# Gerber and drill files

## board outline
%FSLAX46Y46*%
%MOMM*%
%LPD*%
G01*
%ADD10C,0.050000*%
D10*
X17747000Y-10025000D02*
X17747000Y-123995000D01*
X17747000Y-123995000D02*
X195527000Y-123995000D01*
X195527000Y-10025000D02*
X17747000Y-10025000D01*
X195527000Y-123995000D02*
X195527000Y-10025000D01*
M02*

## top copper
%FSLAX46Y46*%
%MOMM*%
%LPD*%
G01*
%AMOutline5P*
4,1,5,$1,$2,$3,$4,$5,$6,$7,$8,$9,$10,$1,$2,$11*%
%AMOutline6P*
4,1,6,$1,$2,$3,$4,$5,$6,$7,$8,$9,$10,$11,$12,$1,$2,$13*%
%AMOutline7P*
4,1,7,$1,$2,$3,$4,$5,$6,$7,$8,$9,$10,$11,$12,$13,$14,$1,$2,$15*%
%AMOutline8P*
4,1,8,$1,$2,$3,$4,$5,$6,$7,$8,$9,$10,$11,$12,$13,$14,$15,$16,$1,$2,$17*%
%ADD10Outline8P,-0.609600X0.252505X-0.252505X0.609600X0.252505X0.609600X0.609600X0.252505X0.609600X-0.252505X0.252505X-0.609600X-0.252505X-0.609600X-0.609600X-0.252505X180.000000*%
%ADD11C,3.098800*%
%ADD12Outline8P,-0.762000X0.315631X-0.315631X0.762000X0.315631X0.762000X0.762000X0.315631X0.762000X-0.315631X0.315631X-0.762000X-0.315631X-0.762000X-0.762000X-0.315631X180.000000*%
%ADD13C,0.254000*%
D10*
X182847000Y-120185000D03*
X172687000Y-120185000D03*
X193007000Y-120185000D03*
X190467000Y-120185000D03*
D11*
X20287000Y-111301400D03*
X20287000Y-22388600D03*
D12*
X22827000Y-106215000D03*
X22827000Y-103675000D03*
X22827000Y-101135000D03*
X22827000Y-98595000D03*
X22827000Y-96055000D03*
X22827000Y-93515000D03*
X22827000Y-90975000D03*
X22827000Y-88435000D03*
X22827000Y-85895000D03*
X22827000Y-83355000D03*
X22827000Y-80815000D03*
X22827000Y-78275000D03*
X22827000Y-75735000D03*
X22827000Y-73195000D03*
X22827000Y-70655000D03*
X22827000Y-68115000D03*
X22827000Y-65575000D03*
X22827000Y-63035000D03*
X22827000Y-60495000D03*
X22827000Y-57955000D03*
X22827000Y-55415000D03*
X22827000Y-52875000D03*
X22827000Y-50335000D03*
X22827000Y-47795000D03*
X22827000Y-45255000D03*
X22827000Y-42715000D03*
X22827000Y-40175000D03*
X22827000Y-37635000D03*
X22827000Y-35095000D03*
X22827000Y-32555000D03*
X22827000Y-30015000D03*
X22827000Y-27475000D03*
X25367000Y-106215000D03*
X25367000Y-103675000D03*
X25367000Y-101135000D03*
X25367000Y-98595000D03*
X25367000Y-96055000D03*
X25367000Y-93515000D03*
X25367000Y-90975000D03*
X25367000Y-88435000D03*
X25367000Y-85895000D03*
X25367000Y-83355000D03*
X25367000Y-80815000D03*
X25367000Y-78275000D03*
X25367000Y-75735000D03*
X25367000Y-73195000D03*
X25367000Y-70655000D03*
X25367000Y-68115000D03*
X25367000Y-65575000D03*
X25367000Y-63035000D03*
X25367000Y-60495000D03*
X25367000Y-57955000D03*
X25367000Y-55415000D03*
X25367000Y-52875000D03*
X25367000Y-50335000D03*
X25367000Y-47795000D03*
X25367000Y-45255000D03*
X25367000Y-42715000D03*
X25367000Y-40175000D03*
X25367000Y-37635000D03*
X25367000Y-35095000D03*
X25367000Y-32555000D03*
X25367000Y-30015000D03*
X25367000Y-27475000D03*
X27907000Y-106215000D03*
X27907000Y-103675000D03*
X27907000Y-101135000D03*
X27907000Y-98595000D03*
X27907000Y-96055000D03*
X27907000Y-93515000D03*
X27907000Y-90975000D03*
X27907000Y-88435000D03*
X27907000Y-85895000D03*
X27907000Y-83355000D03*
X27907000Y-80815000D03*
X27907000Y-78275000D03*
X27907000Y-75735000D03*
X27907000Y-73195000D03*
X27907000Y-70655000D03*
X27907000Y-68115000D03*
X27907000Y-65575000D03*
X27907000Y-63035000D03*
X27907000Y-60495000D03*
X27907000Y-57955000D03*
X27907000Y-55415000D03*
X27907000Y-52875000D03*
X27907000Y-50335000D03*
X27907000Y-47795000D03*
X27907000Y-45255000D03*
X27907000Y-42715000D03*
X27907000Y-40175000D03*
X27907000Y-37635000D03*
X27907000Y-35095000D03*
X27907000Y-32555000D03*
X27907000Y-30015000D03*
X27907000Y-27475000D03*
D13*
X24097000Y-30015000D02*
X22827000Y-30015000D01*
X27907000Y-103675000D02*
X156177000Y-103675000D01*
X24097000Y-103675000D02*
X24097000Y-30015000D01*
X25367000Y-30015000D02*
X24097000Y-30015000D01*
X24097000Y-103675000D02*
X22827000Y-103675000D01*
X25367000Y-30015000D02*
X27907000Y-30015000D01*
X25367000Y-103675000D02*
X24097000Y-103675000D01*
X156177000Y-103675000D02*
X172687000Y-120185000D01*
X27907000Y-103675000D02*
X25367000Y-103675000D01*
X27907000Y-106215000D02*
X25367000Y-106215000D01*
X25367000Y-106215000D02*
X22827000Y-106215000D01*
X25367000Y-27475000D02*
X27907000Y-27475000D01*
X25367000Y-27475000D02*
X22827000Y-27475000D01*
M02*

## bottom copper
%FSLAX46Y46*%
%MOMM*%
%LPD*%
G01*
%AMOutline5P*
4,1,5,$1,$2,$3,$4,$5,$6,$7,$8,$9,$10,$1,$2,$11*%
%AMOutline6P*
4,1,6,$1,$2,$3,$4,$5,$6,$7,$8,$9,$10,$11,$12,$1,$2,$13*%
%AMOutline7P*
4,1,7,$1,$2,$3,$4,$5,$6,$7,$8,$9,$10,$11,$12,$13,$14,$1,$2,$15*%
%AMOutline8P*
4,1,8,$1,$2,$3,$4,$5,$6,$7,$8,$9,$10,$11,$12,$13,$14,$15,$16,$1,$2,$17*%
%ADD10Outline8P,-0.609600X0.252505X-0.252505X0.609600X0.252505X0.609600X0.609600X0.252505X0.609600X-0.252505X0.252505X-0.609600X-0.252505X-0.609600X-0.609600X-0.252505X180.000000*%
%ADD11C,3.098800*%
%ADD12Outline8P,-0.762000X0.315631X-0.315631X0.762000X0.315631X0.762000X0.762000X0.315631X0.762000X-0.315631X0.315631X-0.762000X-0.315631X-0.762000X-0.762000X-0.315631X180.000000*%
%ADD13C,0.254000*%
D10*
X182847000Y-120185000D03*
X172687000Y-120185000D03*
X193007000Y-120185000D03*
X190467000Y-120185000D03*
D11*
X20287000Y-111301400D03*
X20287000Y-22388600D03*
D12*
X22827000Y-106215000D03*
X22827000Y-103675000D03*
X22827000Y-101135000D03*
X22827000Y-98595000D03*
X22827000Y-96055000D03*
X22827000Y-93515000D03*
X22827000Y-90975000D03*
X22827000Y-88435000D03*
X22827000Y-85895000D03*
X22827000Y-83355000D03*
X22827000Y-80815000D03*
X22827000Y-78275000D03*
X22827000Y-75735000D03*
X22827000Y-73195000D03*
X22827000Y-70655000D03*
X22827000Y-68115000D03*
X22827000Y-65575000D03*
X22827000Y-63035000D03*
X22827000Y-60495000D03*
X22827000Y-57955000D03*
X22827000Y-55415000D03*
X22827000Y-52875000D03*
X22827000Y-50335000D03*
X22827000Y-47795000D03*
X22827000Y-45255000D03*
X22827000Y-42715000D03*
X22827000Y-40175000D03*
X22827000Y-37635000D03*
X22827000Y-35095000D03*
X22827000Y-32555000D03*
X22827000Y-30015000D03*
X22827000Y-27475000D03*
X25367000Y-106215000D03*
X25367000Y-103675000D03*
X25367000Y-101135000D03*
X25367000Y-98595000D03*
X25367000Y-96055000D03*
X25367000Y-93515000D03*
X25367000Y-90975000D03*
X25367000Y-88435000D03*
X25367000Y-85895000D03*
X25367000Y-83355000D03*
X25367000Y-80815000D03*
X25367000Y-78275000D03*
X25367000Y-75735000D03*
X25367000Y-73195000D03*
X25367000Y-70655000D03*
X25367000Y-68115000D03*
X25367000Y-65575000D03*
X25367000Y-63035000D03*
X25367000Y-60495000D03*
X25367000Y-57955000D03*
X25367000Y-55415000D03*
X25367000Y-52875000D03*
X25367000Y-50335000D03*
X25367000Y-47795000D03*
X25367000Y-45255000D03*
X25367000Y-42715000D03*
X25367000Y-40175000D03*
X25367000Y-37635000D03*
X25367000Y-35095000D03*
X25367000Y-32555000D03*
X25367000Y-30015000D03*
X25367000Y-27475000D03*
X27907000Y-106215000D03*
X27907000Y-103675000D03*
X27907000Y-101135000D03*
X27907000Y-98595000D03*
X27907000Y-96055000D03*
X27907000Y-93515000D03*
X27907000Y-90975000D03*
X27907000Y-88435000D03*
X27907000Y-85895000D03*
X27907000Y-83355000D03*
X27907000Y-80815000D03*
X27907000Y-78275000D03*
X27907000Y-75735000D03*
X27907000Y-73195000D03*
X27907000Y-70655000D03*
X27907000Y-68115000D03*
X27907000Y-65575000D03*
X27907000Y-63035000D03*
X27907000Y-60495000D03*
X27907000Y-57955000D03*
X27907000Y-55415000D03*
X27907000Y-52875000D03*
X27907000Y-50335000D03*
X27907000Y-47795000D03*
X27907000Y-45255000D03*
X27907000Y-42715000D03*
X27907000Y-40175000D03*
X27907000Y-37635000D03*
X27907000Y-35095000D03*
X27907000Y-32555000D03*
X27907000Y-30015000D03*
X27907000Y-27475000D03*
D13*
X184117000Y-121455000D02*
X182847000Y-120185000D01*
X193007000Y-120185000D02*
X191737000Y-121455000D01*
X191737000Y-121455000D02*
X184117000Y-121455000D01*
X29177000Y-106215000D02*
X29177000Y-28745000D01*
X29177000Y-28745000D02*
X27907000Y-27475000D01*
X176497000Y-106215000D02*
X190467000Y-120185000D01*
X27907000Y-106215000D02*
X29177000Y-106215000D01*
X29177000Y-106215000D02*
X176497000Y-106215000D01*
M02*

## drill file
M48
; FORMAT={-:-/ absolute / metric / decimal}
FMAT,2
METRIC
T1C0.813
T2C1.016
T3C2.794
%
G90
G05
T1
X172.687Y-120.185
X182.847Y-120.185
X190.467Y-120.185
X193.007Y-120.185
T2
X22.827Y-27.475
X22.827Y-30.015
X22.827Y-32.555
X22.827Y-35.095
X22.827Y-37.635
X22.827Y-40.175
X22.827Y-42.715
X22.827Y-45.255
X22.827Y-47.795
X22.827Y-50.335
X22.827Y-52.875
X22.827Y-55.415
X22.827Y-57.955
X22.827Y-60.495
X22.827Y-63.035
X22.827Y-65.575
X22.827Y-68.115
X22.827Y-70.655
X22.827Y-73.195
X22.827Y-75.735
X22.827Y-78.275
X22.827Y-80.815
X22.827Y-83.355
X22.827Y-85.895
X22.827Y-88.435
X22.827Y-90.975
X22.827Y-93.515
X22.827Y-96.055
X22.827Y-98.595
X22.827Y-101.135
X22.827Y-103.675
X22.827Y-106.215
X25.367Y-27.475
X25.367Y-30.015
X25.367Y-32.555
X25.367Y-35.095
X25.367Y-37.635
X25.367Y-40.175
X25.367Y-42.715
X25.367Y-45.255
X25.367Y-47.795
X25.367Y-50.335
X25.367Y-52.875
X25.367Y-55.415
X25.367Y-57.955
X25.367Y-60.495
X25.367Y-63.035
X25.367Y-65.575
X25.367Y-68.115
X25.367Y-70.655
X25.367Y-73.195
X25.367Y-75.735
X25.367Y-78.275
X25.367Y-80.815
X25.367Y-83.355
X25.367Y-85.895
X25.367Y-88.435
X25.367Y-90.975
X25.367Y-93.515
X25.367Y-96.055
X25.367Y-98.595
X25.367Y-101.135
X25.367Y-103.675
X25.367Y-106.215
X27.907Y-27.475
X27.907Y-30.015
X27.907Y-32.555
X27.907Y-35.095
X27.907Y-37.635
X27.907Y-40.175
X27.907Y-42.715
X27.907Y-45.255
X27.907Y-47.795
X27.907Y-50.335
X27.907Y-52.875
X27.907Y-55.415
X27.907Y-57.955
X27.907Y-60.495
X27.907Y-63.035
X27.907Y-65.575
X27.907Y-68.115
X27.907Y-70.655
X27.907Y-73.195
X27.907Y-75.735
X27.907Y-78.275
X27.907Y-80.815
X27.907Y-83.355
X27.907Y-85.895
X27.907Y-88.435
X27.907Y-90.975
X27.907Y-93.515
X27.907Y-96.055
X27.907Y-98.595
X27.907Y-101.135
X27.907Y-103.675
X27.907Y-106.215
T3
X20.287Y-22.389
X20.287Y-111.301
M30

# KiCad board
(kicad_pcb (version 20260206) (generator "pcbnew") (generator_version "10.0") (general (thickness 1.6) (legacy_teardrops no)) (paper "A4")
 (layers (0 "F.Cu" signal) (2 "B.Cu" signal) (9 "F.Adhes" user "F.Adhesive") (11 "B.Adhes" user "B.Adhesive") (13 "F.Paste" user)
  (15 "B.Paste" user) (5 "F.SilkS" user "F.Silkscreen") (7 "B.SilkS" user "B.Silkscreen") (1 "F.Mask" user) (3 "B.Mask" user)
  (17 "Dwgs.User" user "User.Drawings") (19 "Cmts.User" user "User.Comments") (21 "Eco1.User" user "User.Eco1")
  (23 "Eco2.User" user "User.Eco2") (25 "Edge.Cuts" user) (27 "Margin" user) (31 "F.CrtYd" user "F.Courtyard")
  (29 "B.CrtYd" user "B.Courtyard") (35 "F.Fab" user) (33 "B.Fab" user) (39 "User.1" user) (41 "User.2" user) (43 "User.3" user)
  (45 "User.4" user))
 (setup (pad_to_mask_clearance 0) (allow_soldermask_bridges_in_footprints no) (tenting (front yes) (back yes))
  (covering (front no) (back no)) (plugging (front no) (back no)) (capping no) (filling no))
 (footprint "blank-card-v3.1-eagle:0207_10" (layer "F.Cu") (at 177.767 120.185 180)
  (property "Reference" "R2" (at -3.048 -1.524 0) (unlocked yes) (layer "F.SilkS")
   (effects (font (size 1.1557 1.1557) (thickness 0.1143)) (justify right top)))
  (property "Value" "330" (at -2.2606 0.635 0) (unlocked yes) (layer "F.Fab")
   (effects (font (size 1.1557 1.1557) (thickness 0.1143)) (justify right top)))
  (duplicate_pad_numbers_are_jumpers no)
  (pad "1" thru_hole roundrect (at -5.08 0 180) (size 1.2192 1.2192) (drill 0.8128) (layers "*.Cu" "*.Mask") (remove_unused_layers no)
   (roundrect_rratio 0.25) (chamfer_ratio 0.2928932188) (chamfer top_left top_right bottom_left bottom_right) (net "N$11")
   (solder_mask_margin 0.0635) (thermal_bridge_angle 0))
  (pad "2" thru_hole roundrect (at 5.08 0 180) (size 1.2192 1.2192) (drill 0.8128) (layers "*.Cu" "*.Mask") (remove_unused_layers no)
   (roundrect_rratio 0.25) (chamfer_ratio 0.2928932188) (chamfer top_left top_right bottom_left bottom_right) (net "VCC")
   (solder_mask_margin 0.0635) (thermal_bridge_angle 0)))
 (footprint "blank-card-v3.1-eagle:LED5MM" (layer "F.Cu") (at 191.737 120.185 180)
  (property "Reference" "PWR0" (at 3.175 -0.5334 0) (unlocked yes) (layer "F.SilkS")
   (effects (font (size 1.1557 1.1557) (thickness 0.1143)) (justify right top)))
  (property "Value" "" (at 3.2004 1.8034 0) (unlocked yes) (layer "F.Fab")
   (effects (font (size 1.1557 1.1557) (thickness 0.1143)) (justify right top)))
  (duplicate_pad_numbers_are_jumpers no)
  (pad "A" thru_hole roundrect (at -1.27 0 180) (size 1.2192 1.2192) (drill 0.8128) (layers "*.Cu" "*.Mask") (remove_unused_layers no)
   (roundrect_rratio 0.25) (chamfer_ratio 0.2928932188) (chamfer top_left top_right bottom_left bottom_right) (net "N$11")
   (solder_mask_margin 0.0635) (thermal_bridge_angle 0))
  (pad "K" thru_hole roundrect (at 1.27 0 180) (size 1.2192 1.2192) (drill 0.8128) (layers "*.Cu" "*.Mask") (remove_unused_layers no)
   (roundrect_rratio 0.25) (chamfer_ratio 0.2928932188) (chamfer top_left top_right bottom_left bottom_right) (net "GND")
   (solder_mask_margin 0.0635) (thermal_bridge_angle 0)))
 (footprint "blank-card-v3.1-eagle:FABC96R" (layer "F.Cu") (at 20.287 66.845 180)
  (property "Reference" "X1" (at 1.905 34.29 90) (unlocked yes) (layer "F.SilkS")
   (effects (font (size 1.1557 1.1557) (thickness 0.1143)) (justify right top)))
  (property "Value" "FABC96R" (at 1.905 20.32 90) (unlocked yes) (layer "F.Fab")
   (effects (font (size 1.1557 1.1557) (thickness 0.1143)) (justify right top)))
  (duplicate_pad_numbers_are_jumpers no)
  (pad "" np_thru_hole circle (at 0 -44.4564 180) (size 3.0988 3.0988) (drill 2.794) (layers "*.Cu" "*.Mask"))
  (pad "" np_thru_hole circle (at 0 44.4564 180) (size 3.0988 3.0988) (drill 2.794) (layers "*.Cu" "*.Mask"))
  (pad "A1" thru_hole roundrect (at -2.54 -39.37 180) (size 1.524 1.524) (drill 1.016) (layers "*.Cu" "*.Mask") (remove_unused_layers no)
   (roundrect_rratio 0.25) (chamfer_ratio 0.2928932188) (chamfer top_left top_right bottom_left bottom_right) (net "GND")
   (solder_mask_margin 0.0635) (thermal_bridge_angle 0))
  (pad "A2" thru_hole roundrect (at -2.54 -36.83 180) (size 1.524 1.524) (drill 1.016) (layers "*.Cu" "*.Mask") (remove_unused_layers no)
   (roundrect_rratio 0.25) (chamfer_ratio 0.2928932188) (chamfer top_left top_right bottom_left bottom_right) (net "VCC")
   (solder_mask_margin 0.0635) (thermal_bridge_angle 0))
  (pad "A3" thru_hole roundrect (at -2.54 -34.29 180) (size 1.524 1.524) (drill 1.016) (layers "*.Cu" "*.Mask") (remove_unused_layers no)
   (roundrect_rratio 0.25) (chamfer_ratio 0.2928932188) (chamfer top_left top_right bottom_left bottom_right) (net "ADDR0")
   (solder_mask_margin 0.0635) (thermal_bridge_angle 0))
  (pad "A4" thru_hole roundrect (at -2.54 -31.75 180) (size 1.524 1.524) (drill 1.016) (layers "*.Cu" "*.Mask") (remove_unused_layers no)
   (roundrect_rratio 0.25) (chamfer_ratio 0.2928932188) (chamfer top_left top_right bottom_left bottom_right) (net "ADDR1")
   (solder_mask_margin 0.0635) (thermal_bridge_angle 0))
  (pad "A5" thru_hole roundrect (at -2.54 -29.21 180) (size 1.524 1.524) (drill 1.016) (layers "*.Cu" "*.Mask") (remove_unused_layers no)
   (roundrect_rratio 0.25) (chamfer_ratio 0.2928932188) (chamfer top_left top_right bottom_left bottom_right) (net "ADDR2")
   (solder_mask_margin 0.0635) (thermal_bridge_angle 0))
  (pad "A6" thru_hole roundrect (at -2.54 -26.67 180) (size 1.524 1.524) (drill 1.016) (layers "*.Cu" "*.Mask") (remove_unused_layers no)
   (roundrect_rratio 0.25) (chamfer_ratio 0.2928932188) (chamfer top_left top_right bottom_left bottom_right) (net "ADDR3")
   (solder_mask_margin 0.0635) (thermal_bridge_angle 0))
  (pad "A7" thru_hole roundrect (at -2.54 -24.13 180) (size 1.524 1.524) (drill 1.016) (layers "*.Cu" "*.Mask") (remove_unused_layers no)
   (roundrect_rratio 0.25) (chamfer_ratio 0.2928932188) (chamfer top_left top_right bottom_left bottom_right) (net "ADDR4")
   (solder_mask_margin 0.0635) (thermal_bridge_angle 0))
  (pad "A8" thru_hole roundrect (at -2.54 -21.59 180) (size 1.524 1.524) (drill 1.016) (layers "*.Cu" "*.Mask") (remove_unused_layers no)
   (roundrect_rratio 0.25) (chamfer_ratio 0.2928932188) (chamfer top_left top_right bottom_left bottom_right) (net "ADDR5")
   (solder_mask_margin 0.0635) (thermal_bridge_angle 0))
  (pad "A9" thru_hole roundrect (at -2.54 -19.05 180) (size 1.524 1.524) (drill 1.016) (layers "*.Cu" "*.Mask") (remove_unused_layers no)
   (roundrect_rratio 0.25) (chamfer_ratio 0.2928932188) (chamfer top_left top_right bottom_left bottom_right) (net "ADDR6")
   (solder_mask_margin 0.0635) (thermal_bridge_angle 0))
  (pad "A10" thru_hole roundrect (at -2.54 -16.51 180) (size 1.524 1.524) (drill 1.016) (layers "*.Cu" "*.Mask") (remove_unused_layers no)
   (roundrect_rratio 0.25) (chamfer_ratio 0.2928932188) (chamfer top_left top_right bottom_left bottom_right) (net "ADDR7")
   (solder_mask_margin 0.0635) (thermal_bridge_angle 0))
  (pad "A11" thru_hole roundrect (at -2.54 -13.97 180) (size 1.524 1.524) (drill 1.016) (layers "*.Cu" "*.Mask") (remove_unused_layers no)
   (roundrect_rratio 0.25) (chamfer_ratio 0.2928932188) (chamfer top_left top_right bottom_left bottom_right) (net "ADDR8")
   (solder_mask_margin 0.0635) (thermal_bridge_angle 0))
  (pad "A12" thru_hole roundrect (at -2.54 -11.43 180) (size 1.524 1.524) (drill 1.016) (layers "*.Cu" "*.Mask") (remove_unused_layers no)
   (roundrect_rratio 0.25) (chamfer_ratio 0.2928932188) (chamfer top_left top_right bottom_left bottom_right) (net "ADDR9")
   (solder_mask_margin 0.0635) (thermal_bridge_angle 0))
  (pad "A13" thru_hole roundrect (at -2.54 -8.89 180) (size 1.524 1.524) (drill 1.016) (layers "*.Cu" "*.Mask") (remove_unused_layers no)
   (roundrect_rratio 0.25) (chamfer_ratio 0.2928932188) (chamfer top_left top_right bottom_left bottom_right) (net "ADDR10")
   (solder_mask_margin 0.0635) (thermal_bridge_angle 0))
  (pad "A14" thru_hole roundrect (at -2.54 -6.35 180) (size 1.524 1.524) (drill 1.016) (layers "*.Cu" "*.Mask") (remove_unused_layers no)
   (roundrect_rratio 0.25) (chamfer_ratio 0.2928932188) (chamfer top_left top_right bottom_left bottom_right) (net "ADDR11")
   (solder_mask_margin 0.0635) (thermal_bridge_angle 0))
  (pad "A15" thru_hole roundrect (at -2.54 -3.81 180) (size 1.524 1.524) (drill 1.016) (layers "*.Cu" "*.Mask") (remove_unused_layers no)
   (roundrect_rratio 0.25) (chamfer_ratio 0.2928932188) (chamfer top_left top_right bottom_left bottom_right) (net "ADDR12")
   (solder_mask_margin 0.0635) (thermal_bridge_angle 0))
  (pad "A16" thru_hole roundrect (at -2.54 -1.27 180) (size 1.524 1.524) (drill 1.016) (layers "*.Cu" "*.Mask") (remove_unused_layers no)
   (roundrect_rratio 0.25) (chamfer_ratio 0.2928932188) (chamfer top_left top_right bottom_left bottom_right) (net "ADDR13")
   (solder_mask_margin 0.0635) (thermal_bridge_angle 0))
  (pad "A17" thru_hole roundrect (at -2.54 1.27 180) (size 1.524 1.524) (drill 1.016) (layers "*.Cu" "*.Mask") (remove_unused_layers no)
   (roundrect_rratio 0.25) (chamfer_ratio 0.2928932188) (chamfer top_left top_right bottom_left bottom_right) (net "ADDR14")
   (solder_mask_margin 0.0635) (thermal_bridge_angle 0))
  (pad "A18" thru_hole roundrect (at -2.54 3.81 180) (size 1.524 1.524) (drill 1.016) (layers "*.Cu" "*.Mask") (remove_unused_layers no)
   (roundrect_rratio 0.25) (chamfer_ratio 0.2928932188) (chamfer top_left top_right bottom_left bottom_right) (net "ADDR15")
   (solder_mask_margin 0.0635) (thermal_bridge_angle 0))
  (pad "A19" thru_hole roundrect (at -2.54 6.35 180) (size 1.524 1.524) (drill 1.016) (layers "*.Cu" "*.Mask") (remove_unused_layers no)
   (roundrect_rratio 0.25) (chamfer_ratio 0.2928932188) (chamfer top_left top_right bottom_left bottom_right) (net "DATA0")
   (solder_mask_margin 0.0635) (thermal_bridge_angle 0))
  (pad "A20" thru_hole roundrect (at -2.54 8.89 180) (size 1.524 1.524) (drill 1.016) (layers "*.Cu" "*.Mask") (remove_unused_layers no)
   (roundrect_rratio 0.25) (chamfer_ratio 0.2928932188) (chamfer top_left top_right bottom_left bottom_right) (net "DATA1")
   (solder_mask_margin 0.0635) (thermal_bridge_angle 0))
  (pad "A21" thru_hole roundrect (at -2.54 11.43 180) (size 1.524 1.524) (drill 1.016) (layers "*.Cu" "*.Mask") (remove_unused_layers no)
   (roundrect_rratio 0.25) (chamfer_ratio 0.2928932188) (chamfer top_left top_right bottom_left bottom_right) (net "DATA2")
   (solder_mask_margin 0.0635) (thermal_bridge_angle 0))
  (pad "A22" thru_hole roundrect (at -2.54 13.97 180) (size 1.524 1.524) (drill 1.016) (layers "*.Cu" "*.Mask") (remove_unused_layers no)
   (roundrect_rratio 0.25) (chamfer_ratio 0.2928932188) (chamfer top_left top_right bottom_left bottom_right) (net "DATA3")
   (solder_mask_margin 0.0635) (thermal_bridge_angle 0))
  (pad "A23" thru_hole roundrect (at -2.54 16.51 180) (size 1.524 1.524) (drill 1.016) (layers "*.Cu" "*.Mask") (remove_unused_layers no)
   (roundrect_rratio 0.25) (chamfer_ratio 0.2928932188) (chamfer top_left top_right bottom_left bottom_right) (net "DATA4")
   (solder_mask_margin 0.0635) (thermal_bridge_angle 0))
  (pad "A24" thru_hole roundrect (at -2.54 19.05 180) (size 1.524 1.524) (drill 1.016) (layers "*.Cu" "*.Mask") (remove_unused_layers no)
   (roundrect_rratio 0.25) (chamfer_ratio 0.2928932188) (chamfer top_left top_right bottom_left bottom_right) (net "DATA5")
   (solder_mask_margin 0.0635) (thermal_bridge_angle 0))
  (pad "A25" thru_hole roundrect (at -2.54 21.59 180) (size 1.524 1.524) (drill 1.016) (layers "*.Cu" "*.Mask") (remove_unused_layers no)
   (roundrect_rratio 0.25) (chamfer_ratio 0.2928932188) (chamfer top_left top_right bottom_left bottom_right) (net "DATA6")
   (solder_mask_margin 0.0635) (thermal_bridge_angle 0))
  (pad "A26" thru_hole roundrect (at -2.54 24.13 180) (size 1.524 1.524) (drill 1.016) (layers "*.Cu" "*.Mask") (remove_unused_layers no)
   (roundrect_rratio 0.25) (chamfer_ratio 0.2928932188) (chamfer top_left top_right bottom_left bottom_right) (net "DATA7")
   (solder_mask_margin 0.0635) (thermal_bridge_angle 0))
  (pad "A27" thru_hole roundrect (at -2.54 26.67 180) (size 1.524 1.524) (drill 1.016) (layers "*.Cu" "*.Mask") (remove_unused_layers no)
   (roundrect_rratio 0.25) (chamfer_ratio 0.2928932188) (chamfer top_left top_right bottom_left bottom_right) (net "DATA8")
   (solder_mask_margin 0.0635) (thermal_bridge_angle 0))
  (pad "A28" thru_hole roundrect (at -2.54 29.21 180) (size 1.524 1.524) (drill 1.016) (layers "*.Cu" "*.Mask") (remove_unused_layers no)
   (roundrect_rratio 0.25) (chamfer_ratio 0.2928932188) (chamfer top_left top_right bottom_left bottom_right) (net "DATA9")
   (solder_mask_margin 0.0635) (thermal_bridge_angle 0))
  (pad "A29" thru_hole roundrect (at -2.54 31.75 180) (size 1.524 1.524) (drill 1.016) (layers "*.Cu" "*.Mask") (remove_unused_layers no)
   (roundrect_rratio 0.25) (chamfer_ratio 0.2928932188) (chamfer top_left top_right bottom_left bottom_right) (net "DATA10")
   (solder_mask_margin 0.0635) (thermal_bridge_angle 0))
  (pad "A30" thru_hole roundrect (at -2.54 34.29 180) (size 1.524 1.524) (drill 1.016) (layers "*.Cu" "*.Mask") (remove_unused_layers no)
   (roundrect_rratio 0.25) (chamfer_ratio 0.2928932188) (chamfer top_left top_right bottom_left bottom_right) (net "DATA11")
   (solder_mask_margin 0.0635) (thermal_bridge_angle 0))
  (pad "A31" thru_hole roundrect (at -2.54 36.83 180) (size 1.524 1.524) (drill 1.016) (layers "*.Cu" "*.Mask") (remove_unused_layers no)
   (roundrect_rratio 0.25) (chamfer_ratio 0.2928932188) (chamfer top_left top_right bottom_left bottom_right) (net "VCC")
   (solder_mask_margin 0.0635) (thermal_bridge_angle 0))
  (pad "A32" thru_hole roundrect (at -2.54 39.37 180) (size 1.524 1.524) (drill 1.016) (layers "*.Cu" "*.Mask") (remove_unused_layers no)
   (roundrect_rratio 0.25) (chamfer_ratio 0.2928932188) (chamfer top_left top_right bottom_left bottom_right) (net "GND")
   (solder_mask_margin 0.0635) (thermal_bridge_angle 0))
  (pad "B1" thru_hole roundrect (at -5.08 -39.37 180) (size 1.524 1.524) (drill 1.016) (layers "*.Cu" "*.Mask") (remove_unused_layers no)
   (roundrect_rratio 0.25) (chamfer_ratio 0.2928932188) (chamfer top_left top_right bottom_left bottom_right) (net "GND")
   (solder_mask_margin 0.0635) (thermal_bridge_angle 0))
  (pad "B2" thru_hole roundrect (at -5.08 -36.83 180) (size 1.524 1.524) (drill 1.016) (layers "*.Cu" "*.Mask") (remove_unused_layers no)
   (roundrect_rratio 0.25) (chamfer_ratio 0.2928932188) (chamfer top_left top_right bottom_left bottom_right) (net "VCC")
   (solder_mask_margin 0.0635) (thermal_bridge_angle 0))
  (pad "B3" thru_hole roundrect (at -5.08 -34.29 180) (size 1.524 1.524) (drill 1.016) (layers "*.Cu" "*.Mask") (remove_unused_layers no)
   (roundrect_rratio 0.25) (chamfer_ratio 0.2928932188) (chamfer top_left top_right bottom_left bottom_right) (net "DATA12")
   (solder_mask_margin 0.0635) (thermal_bridge_angle 0))
  (pad "B4" thru_hole roundrect (at -5.08 -31.75 180) (size 1.524 1.524) (drill 1.016) (layers "*.Cu" "*.Mask") (remove_unused_layers no)
   (roundrect_rratio 0.25) (chamfer_ratio 0.2928932188) (chamfer top_left top_right bottom_left bottom_right) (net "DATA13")
   (solder_mask_margin 0.0635) (thermal_bridge_angle 0))
  (pad "B5" thru_hole roundrect (at -5.08 -29.21 180) (size 1.524 1.524) (drill 1.016) (layers "*.Cu" "*.Mask") (remove_unused_layers no)
   (roundrect_rratio 0.25) (chamfer_ratio 0.2928932188) (chamfer top_left top_right bottom_left bottom_right) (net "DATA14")
   (solder_mask_margin 0.0635) (thermal_bridge_angle 0))
  (pad "B6" thru_hole roundrect (at -5.08 -26.67 180) (size 1.524 1.524) (drill 1.016) (layers "*.Cu" "*.Mask") (remove_unused_layers no)
   (roundrect_rratio 0.25) (chamfer_ratio 0.2928932188) (chamfer top_left top_right bottom_left bottom_right) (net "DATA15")
   (solder_mask_margin 0.0635) (thermal_bridge_angle 0))
  (pad "B7" thru_hole roundrect (at -5.08 -24.13 180) (size 1.524 1.524) (drill 1.016) (layers "*.Cu" "*.Mask") (remove_unused_layers no)
   (roundrect_rratio 0.25) (chamfer_ratio 0.2928932188) (chamfer top_left top_right bottom_left bottom_right) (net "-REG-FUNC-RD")
   (solder_mask_margin 0.0635) (thermal_bridge_angle 0))
  (pad "B8" thru_hole roundrect (at -5.08 -21.59 180) (size 1.524 1.524) (drill 1.016) (layers "*.Cu" "*.Mask") (remove_unused_layers no)
   (roundrect_rratio 0.25) (chamfer_ratio 0.2928932188) (chamfer top_left top_right bottom_left bottom_right) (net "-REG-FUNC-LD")
   (solder_mask_margin 0.0635) (thermal_bridge_angle 0))
  (pad "B9" thru_hole roundrect (at -5.08 -19.05 180) (size 1.524 1.524) (drill 1.016) (layers "*.Cu" "*.Mask") (remove_unused_layers no)
   (roundrect_rratio 0.25) (chamfer_ratio 0.2928932188) (chamfer top_left top_right bottom_left bottom_right) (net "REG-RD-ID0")
   (solder_mask_margin 0.0635) (thermal_bridge_angle 0))
  (pad "B10" thru_hole roundrect (at -5.08 -16.51 180) (size 1.524 1.524) (drill 1.016) (layers "*.Cu" "*.Mask") (remove_unused_layers no)
   (roundrect_rratio 0.25) (chamfer_ratio 0.2928932188) (chamfer top_left top_right bottom_left bottom_right) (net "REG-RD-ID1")
   (solder_mask_margin 0.0635) (thermal_bridge_angle 0))
  (pad "B11" thru_hole roundrect (at -5.08 -13.97 180) (size 1.524 1.524) (drill 1.016) (layers "*.Cu" "*.Mask") (remove_unused_layers no)
   (roundrect_rratio 0.25) (chamfer_ratio 0.2928932188) (chamfer top_left top_right bottom_left bottom_right) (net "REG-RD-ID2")
   (solder_mask_margin 0.0635) (thermal_bridge_angle 0))
  (pad "B12" thru_hole roundrect (at -5.08 -11.43 180) (size 1.524 1.524) (drill 1.016) (layers "*.Cu" "*.Mask") (remove_unused_layers no)
   (roundrect_rratio 0.25) (chamfer_ratio 0.2928932188) (chamfer top_left top_right bottom_left bottom_right) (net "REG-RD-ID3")
   (solder_mask_margin 0.0635) (thermal_bridge_angle 0))
  (pad "B13" thru_hole roundrect (at -5.08 -8.89 180) (size 1.524 1.524) (drill 1.016) (layers "*.Cu" "*.Mask") (remove_unused_layers no)
   (roundrect_rratio 0.25) (chamfer_ratio 0.2928932188) (chamfer top_left top_right bottom_left bottom_right) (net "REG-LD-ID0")
   (solder_mask_margin 0.0635) (thermal_bridge_angle 0))
  (pad "B14" thru_hole roundrect (at -5.08 -6.35 180) (size 1.524 1.524) (drill 1.016) (layers "*.Cu" "*.Mask") (remove_unused_layers no)
   (roundrect_rratio 0.25) (chamfer_ratio 0.2928932188) (chamfer top_left top_right bottom_left bottom_right) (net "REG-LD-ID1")
   (solder_mask_margin 0.0635) (thermal_bridge_angle 0))
  (pad "B15" thru_hole roundrect (at -5.08 -3.81 180) (size 1.524 1.524) (drill 1.016) (layers "*.Cu" "*.Mask") (remove_unused_layers no)
   (roundrect_rratio 0.25) (chamfer_ratio 0.2928932188) (chamfer top_left top_right bottom_left bottom_right) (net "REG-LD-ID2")
   (solder_mask_margin 0.0635) (thermal_bridge_angle 0))
  (pad "B16" thru_hole roundrect (at -5.08 -1.27 180) (size 1.524 1.524) (drill 1.016) (layers "*.Cu" "*.Mask") (remove_unused_layers no)
   (roundrect_rratio 0.25) (chamfer_ratio 0.2928932188) (chamfer top_left top_right bottom_left bottom_right) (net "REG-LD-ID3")
   (solder_mask_margin 0.0635) (thermal_bridge_angle 0))
  (pad "B17" thru_hole roundrect (at -5.08 1.27 180) (size 1.524 1.524) (drill 1.016) (layers "*.Cu" "*.Mask") (remove_unused_layers no)
   (roundrect_rratio 0.25) (chamfer_ratio 0.2928932188) (chamfer top_left top_right bottom_left bottom_right) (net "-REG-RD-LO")
   (solder_mask_margin 0.0635) (thermal_bridge_angle 0))
  (pad "B18" thru_hole roundrect (at -5.08 3.81 180) (size 1.524 1.524) (drill 1.016) (layers "*.Cu" "*.Mask") (remove_unused_layers no)
   (roundrect_rratio 0.25) (chamfer_ratio 0.2928932188) (chamfer top_left top_right bottom_left bottom_right) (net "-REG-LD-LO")
   (solder_mask_margin 0.0635) (thermal_bridge_angle 0))
  (pad "B19" thru_hole roundrect (at -5.08 6.35 180) (size 1.524 1.524) (drill 1.016) (layers "*.Cu" "*.Mask") (remove_unused_layers no)
   (roundrect_rratio 0.25) (chamfer_ratio 0.2928932188) (chamfer top_left top_right bottom_left bottom_right) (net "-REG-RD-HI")
   (solder_mask_margin 0.0635) (thermal_bridge_angle 0))
  (pad "B20" thru_hole roundrect (at -5.08 8.89 180) (size 1.524 1.524) (drill 1.016) (layers "*.Cu" "*.Mask") (remove_unused_layers no)
   (roundrect_rratio 0.25) (chamfer_ratio 0.2928932188) (chamfer top_left top_right bottom_left bottom_right) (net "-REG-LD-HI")
   (solder_mask_margin 0.0635) (thermal_bridge_angle 0))
  (pad "B21" thru_hole roundrect (at -5.08 11.43 180) (size 1.524 1.524) (drill 1.016) (layers "*.Cu" "*.Mask") (remove_unused_layers no)
   (roundrect_rratio 0.25) (chamfer_ratio 0.2928932188) (chamfer top_left top_right bottom_left bottom_right) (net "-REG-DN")
   (solder_mask_margin 0.0635) (thermal_bridge_angle 0))
  (pad "B22" thru_hole roundrect (at -5.08 13.97 180) (size 1.524 1.524) (drill 1.016) (layers "*.Cu" "*.Mask") (remove_unused_layers no)
   (roundrect_rratio 0.25) (chamfer_ratio 0.2928932188) (chamfer top_left top_right bottom_left bottom_right) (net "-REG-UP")
   (solder_mask_margin 0.0635) (thermal_bridge_angle 0))
  (pad "B23" thru_hole roundrect (at -5.08 16.51 180) (size 1.524 1.524) (drill 1.016) (layers "*.Cu" "*.Mask") (remove_unused_layers no)
   (roundrect_rratio 0.25) (chamfer_ratio 0.2928932188) (chamfer top_left top_right bottom_left bottom_right) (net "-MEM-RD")
   (solder_mask_margin 0.0635) (thermal_bridge_angle 0))
  (pad "B24" thru_hole roundrect (at -5.08 19.05 180) (size 1.524 1.524) (drill 1.016) (layers "*.Cu" "*.Mask") (remove_unused_layers no)
   (roundrect_rratio 0.25) (chamfer_ratio 0.2928932188) (chamfer top_left top_right bottom_left bottom_right) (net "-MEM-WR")
   (solder_mask_margin 0.0635) (thermal_bridge_angle 0))
  (pad "B25" thru_hole roundrect (at -5.08 21.59 180) (size 1.524 1.524) (drill 1.016) (layers "*.Cu" "*.Mask") (remove_unused_layers no)
   (roundrect_rratio 0.25) (chamfer_ratio 0.2928932188) (chamfer top_left top_right bottom_left bottom_right) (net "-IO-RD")
   (solder_mask_margin 0.0635) (thermal_bridge_angle 0))
  (pad "B26" thru_hole roundrect (at -5.08 24.13 180) (size 1.524 1.524) (drill 1.016) (layers "*.Cu" "*.Mask") (remove_unused_layers no)
   (roundrect_rratio 0.25) (chamfer_ratio 0.2928932188) (chamfer top_left top_right bottom_left bottom_right) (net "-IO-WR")
   (solder_mask_margin 0.0635) (thermal_bridge_angle 0))
  (pad "B27" thru_hole roundrect (at -5.08 26.67 180) (size 1.524 1.524) (drill 1.016) (layers "*.Cu" "*.Mask") (remove_unused_layers no)
   (roundrect_rratio 0.25) (chamfer_ratio 0.2928932188) (chamfer top_left top_right bottom_left bottom_right) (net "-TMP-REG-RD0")
   (solder_mask_margin 0.0635) (thermal_bridge_angle 0))
  (pad "B28" thru_hole roundrect (at -5.08 29.21 180) (size 1.524 1.524) (drill 1.016) (layers "*.Cu" "*.Mask") (remove_unused_layers no)
   (roundrect_rratio 0.25) (chamfer_ratio 0.2928932188) (chamfer top_left top_right bottom_left bottom_right) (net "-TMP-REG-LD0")
   (solder_mask_margin 0.0635) (thermal_bridge_angle 0))
  (pad "B29" thru_hole roundrect (at -5.08 31.75 180) (size 1.524 1.524) (drill 1.016) (layers "*.Cu" "*.Mask") (remove_unused_layers no)
   (roundrect_rratio 0.25) (chamfer_ratio 0.2928932188) (chamfer top_left top_right bottom_left bottom_right) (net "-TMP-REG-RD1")
   (solder_mask_margin 0.0635) (thermal_bridge_angle 0))
  (pad "B30" thru_hole roundrect (at -5.08 34.29 180) (size 1.524 1.524) (drill 1.016) (layers "*.Cu" "*.Mask") (remove_unused_layers no)
   (roundrect_rratio 0.25) (chamfer_ratio 0.2928932188) (chamfer top_left top_right bottom_left bottom_right) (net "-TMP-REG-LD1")
   (solder_mask_margin 0.0635) (thermal_bridge_angle 0))
  (pad "B31" thru_hole roundrect (at -5.08 36.83 180) (size 1.524 1.524) (drill 1.016) (layers "*.Cu" "*.Mask") (remove_unused_layers no)
   (roundrect_rratio 0.25) (chamfer_ratio 0.2928932188) (chamfer top_left top_right bottom_left bottom_right) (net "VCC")
   (solder_mask_margin 0.0635) (thermal_bridge_angle 0))
  (pad "B32" thru_hole roundrect (at -5.08 39.37 180) (size 1.524 1.524) (drill 1.016) (layers "*.Cu" "*.Mask") (remove_unused_layers no)
   (roundrect_rratio 0.25) (chamfer_ratio 0.2928932188) (chamfer top_left top_right bottom_left bottom_right) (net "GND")
   (solder_mask_margin 0.0635) (thermal_bridge_angle 0))
  (pad "C1" thru_hole roundrect (at -7.62 -39.37 180) (size 1.524 1.524) (drill 1.016) (layers "*.Cu" "*.Mask") (remove_unused_layers no)
   (roundrect_rratio 0.25) (chamfer_ratio 0.2928932188) (chamfer top_left top_right bottom_left bottom_right) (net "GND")
   (solder_mask_margin 0.0635) (thermal_bridge_angle 0))
  (pad "C2" thru_hole roundrect (at -7.62 -36.83 180) (size 1.524 1.524) (drill 1.016) (layers "*.Cu" "*.Mask") (remove_unused_layers no)
   (roundrect_rratio 0.25) (chamfer_ratio 0.2928932188) (chamfer top_left top_right bottom_left bottom_right) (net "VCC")
   (solder_mask_margin 0.0635) (thermal_bridge_angle 0))
  (pad "C3" thru_hole roundrect (at -7.62 -34.29 180) (size 1.524 1.524) (drill 1.016) (layers "*.Cu" "*.Mask") (remove_unused_layers no)
   (roundrect_rratio 0.25) (chamfer_ratio 0.2928932188) (chamfer top_left top_right bottom_left bottom_right) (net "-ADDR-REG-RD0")
   (solder_mask_margin 0.0635) (thermal_bridge_angle 0))
  (pad "C4" thru_hole roundrect (at -7.62 -31.75 180) (size 1.524 1.524) (drill 1.016) (layers "*.Cu" "*.Mask") (remove_unused_layers no)
   (roundrect_rratio 0.25) (chamfer_ratio 0.2928932188) (chamfer top_left top_right bottom_left bottom_right) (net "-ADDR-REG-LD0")
   (solder_mask_margin 0.0635) (thermal_bridge_angle 0))
  (pad "C5" thru_hole roundrect (at -7.62 -29.21 180) (size 1.524 1.524) (drill 1.016) (layers "*.Cu" "*.Mask") (remove_unused_layers no)
   (roundrect_rratio 0.25) (chamfer_ratio 0.2928932188) (chamfer top_left top_right bottom_left bottom_right) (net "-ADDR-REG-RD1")
   (solder_mask_margin 0.0635) (thermal_bridge_angle 0))
  (pad "C6" thru_hole roundrect (at -7.62 -26.67 180) (size 1.524 1.524) (drill 1.016) (layers "*.Cu" "*.Mask") (remove_unused_layers no)
   (roundrect_rratio 0.25) (chamfer_ratio 0.2928932188) (chamfer top_left top_right bottom_left bottom_right) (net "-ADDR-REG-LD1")
   (solder_mask_margin 0.0635) (thermal_bridge_angle 0))
  (pad "C7" thru_hole roundrect (at -7.62 -24.13 180) (size 1.524 1.524) (drill 1.016) (layers "*.Cu" "*.Mask") (remove_unused_layers no)
   (roundrect_rratio 0.25) (chamfer_ratio 0.2928932188) (chamfer top_left top_right bottom_left bottom_right) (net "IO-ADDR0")
   (solder_mask_margin 0.0635) (thermal_bridge_angle 0))
  (pad "C8" thru_hole roundrect (at -7.62 -21.59 180) (size 1.524 1.524) (drill 1.016) (layers "*.Cu" "*.Mask") (remove_unused_layers no)
   (roundrect_rratio 0.25) (chamfer_ratio 0.2928932188) (chamfer top_left top_right bottom_left bottom_right) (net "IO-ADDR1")
   (solder_mask_margin 0.0635) (thermal_bridge_angle 0))
  (pad "C9" thru_hole roundrect (at -7.62 -19.05 180) (size 1.524 1.524) (drill 1.016) (layers "*.Cu" "*.Mask") (remove_unused_layers no)
   (roundrect_rratio 0.25) (chamfer_ratio 0.2928932188) (chamfer top_left top_right bottom_left bottom_right) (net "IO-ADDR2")
   (solder_mask_margin 0.0635) (thermal_bridge_angle 0))
  (pad "C10" thru_hole roundrect (at -7.62 -16.51 180) (size 1.524 1.524) (drill 1.016) (layers "*.Cu" "*.Mask") (remove_unused_layers no)
   (roundrect_rratio 0.25) (chamfer_ratio 0.2928932188) (chamfer top_left top_right bottom_left bottom_right) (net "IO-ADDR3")
   (solder_mask_margin 0.0635) (thermal_bridge_angle 0))
  (pad "C11" thru_hole roundrect (at -7.62 -13.97 180) (size 1.524 1.524) (drill 1.016) (layers "*.Cu" "*.Mask") (remove_unused_layers no)
   (roundrect_rratio 0.25) (chamfer_ratio 0.2928932188) (chamfer top_left top_right bottom_left bottom_right) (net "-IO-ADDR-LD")
   (solder_mask_margin 0.0635) (thermal_bridge_angle 0))
  (pad "C12" thru_hole roundrect (at -7.62 -11.43 180) (size 1.524 1.524) (drill 1.016) (layers "*.Cu" "*.Mask") (remove_unused_layers no)
   (roundrect_rratio 0.25) (chamfer_ratio 0.2928932188) (chamfer top_left top_right bottom_left bottom_right) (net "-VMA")
   (solder_mask_margin 0.0635) (thermal_bridge_angle 0))
  (pad "C13" thru_hole roundrect (at -7.62 -8.89 180) (size 1.524 1.524) (drill 1.016) (layers "*.Cu" "*.Mask") (remove_unused_layers no)
   (roundrect_rratio 0.25) (chamfer_ratio 0.2928932188) (chamfer top_left top_right bottom_left bottom_right) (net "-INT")
   (solder_mask_margin 0.0635) (thermal_bridge_angle 0))
  (pad "C14" thru_hole roundrect (at -7.62 -6.35 180) (size 1.524 1.524) (drill 1.016) (layers "*.Cu" "*.Mask") (remove_unused_layers no)
   (roundrect_rratio 0.25) (chamfer_ratio 0.2928932188) (chamfer top_left top_right bottom_left bottom_right) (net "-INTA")
   (solder_mask_margin 0.0635) (thermal_bridge_angle 0))
  (pad "C15" thru_hole roundrect (at -7.62 -3.81 180) (size 1.524 1.524) (drill 1.016) (layers "*.Cu" "*.Mask") (remove_unused_layers no)
   (roundrect_rratio 0.25) (chamfer_ratio 0.2928932188) (chamfer top_left top_right bottom_left bottom_right) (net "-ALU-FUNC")
   (solder_mask_margin 0.0635) (thermal_bridge_angle 0))
  (pad "C16" thru_hole roundrect (at -7.62 -1.27 180) (size 1.524 1.524) (drill 1.016) (layers "*.Cu" "*.Mask") (remove_unused_layers no)
   (roundrect_rratio 0.25) (chamfer_ratio 0.2928932188) (chamfer top_left top_right bottom_left bottom_right) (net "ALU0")
   (solder_mask_margin 0.0635) (thermal_bridge_angle 0))
  (pad "C17" thru_hole roundrect (at -7.62 1.27 180) (size 1.524 1.524) (drill 1.016) (layers "*.Cu" "*.Mask") (remove_unused_layers no)
   (roundrect_rratio 0.25) (chamfer_ratio 0.2928932188) (chamfer top_left top_right bottom_left bottom_right) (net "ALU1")
   (solder_mask_margin 0.0635) (thermal_bridge_angle 0))
  (pad "C18" thru_hole roundrect (at -7.62 3.81 180) (size 1.524 1.524) (drill 1.016) (layers "*.Cu" "*.Mask") (remove_unused_layers no)
   (roundrect_rratio 0.25) (chamfer_ratio 0.2928932188) (chamfer top_left top_right bottom_left bottom_right) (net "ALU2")
   (solder_mask_margin 0.0635) (thermal_bridge_angle 0))
  (pad "C19" thru_hole roundrect (at -7.62 6.35 180) (size 1.524 1.524) (drill 1.016) (layers "*.Cu" "*.Mask") (remove_unused_layers no)
   (roundrect_rratio 0.25) (chamfer_ratio 0.2928932188) (chamfer top_left top_right bottom_left bottom_right) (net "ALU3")
   (solder_mask_margin 0.0635) (thermal_bridge_angle 0))
  (pad "C20" thru_hole roundrect (at -7.62 8.89 180) (size 1.524 1.524) (drill 1.016) (layers "*.Cu" "*.Mask") (remove_unused_layers no)
   (roundrect_rratio 0.25) (chamfer_ratio 0.2928932188) (chamfer top_left top_right bottom_left bottom_right) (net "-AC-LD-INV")
   (solder_mask_margin 0.0635) (thermal_bridge_angle 0))
  (pad "C21" thru_hole roundrect (at -7.62 11.43 180) (size 1.524 1.524) (drill 1.016) (layers "*.Cu" "*.Mask") (remove_unused_layers no)
   (roundrect_rratio 0.25) (chamfer_ratio 0.2928932188) (chamfer top_left top_right bottom_left bottom_right) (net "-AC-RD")
   (solder_mask_margin 0.0635) (thermal_bridge_angle 0))
  (pad "C22" thru_hole roundrect (at -7.62 13.97 180) (size 1.524 1.524) (drill 1.016) (layers "*.Cu" "*.Mask") (remove_unused_layers no)
   (roundrect_rratio 0.25) (chamfer_ratio 0.2928932188) (chamfer top_left top_right bottom_left bottom_right) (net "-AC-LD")
   (solder_mask_margin 0.0635) (thermal_bridge_angle 0))
  (pad "C23" thru_hole roundrect (at -7.62 16.51 180) (size 1.524 1.524) (drill 1.016) (layers "*.Cu" "*.Mask") (remove_unused_layers no)
   (roundrect_rratio 0.25) (chamfer_ratio 0.2928932188) (chamfer top_left top_right bottom_left bottom_right) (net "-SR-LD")
   (solder_mask_margin 0.0635) (thermal_bridge_angle 0))
  (pad "C24" thru_hole roundrect (at -7.62 19.05 180) (size 1.524 1.524) (drill 1.016) (layers "*.Cu" "*.Mask") (remove_unused_layers no)
   (roundrect_rratio 0.25) (chamfer_ratio 0.2928932188) (chamfer top_left top_right bottom_left bottom_right) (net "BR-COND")
   (solder_mask_margin 0.0635) (thermal_bridge_angle 0))
  (pad "C25" thru_hole roundrect (at -7.62 21.59 180) (size 1.524 1.524) (drill 1.016) (layers "*.Cu" "*.Mask") (remove_unused_layers no)
   (roundrect_rratio 0.25) (chamfer_ratio 0.2928932188) (chamfer top_left top_right bottom_left bottom_right) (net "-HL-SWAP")
   (solder_mask_margin 0.0635) (thermal_bridge_angle 0))
  (pad "C26" thru_hole roundrect (at -7.62 24.13 180) (size 1.524 1.524) (drill 1.016) (layers "*.Cu" "*.Mask") (remove_unused_layers no)
   (roundrect_rratio 0.25) (chamfer_ratio 0.2928932188) (chamfer top_left top_right bottom_left bottom_right) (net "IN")
   (solder_mask_margin 0.0635) (thermal_bridge_angle 0))
  (pad "C27" thru_hole roundrect (at -7.62 26.67 180) (size 1.524 1.524) (drill 1.016) (layers "*.Cu" "*.Mask") (remove_unused_layers no)
   (roundrect_rratio 0.25) (chamfer_ratio 0.2928932188) (chamfer top_left top_right bottom_left bottom_right) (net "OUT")
   (solder_mask_margin 0.0635) (thermal_bridge_angle 0))
  (pad "C28" thru_hole roundrect (at -7.62 29.21 180) (size 1.524 1.524) (drill 1.016) (layers "*.Cu" "*.Mask") (remove_unused_layers no)
   (roundrect_rratio 0.25) (chamfer_ratio 0.2928932188) (chamfer top_left top_right bottom_left bottom_right) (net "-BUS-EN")
   (solder_mask_margin 0.0635) (thermal_bridge_angle 0))
  (pad "C29" thru_hole roundrect (at -7.62 31.75 180) (size 1.524 1.524) (drill 1.016) (layers "*.Cu" "*.Mask") (remove_unused_layers no)
   (roundrect_rratio 0.25) (chamfer_ratio 0.2928932188) (chamfer top_left top_right bottom_left bottom_right) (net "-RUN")
   (solder_mask_margin 0.0635) (thermal_bridge_angle 0))
  (pad "C30" thru_hole roundrect (at -7.62 34.29 180) (size 1.524 1.524) (drill 1.016) (layers "*.Cu" "*.Mask") (remove_unused_layers no)
   (roundrect_rratio 0.25) (chamfer_ratio 0.2928932188) (chamfer top_left top_right bottom_left bottom_right) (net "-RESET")
   (solder_mask_margin 0.0635) (thermal_bridge_angle 0))
  (pad "C31" thru_hole roundrect (at -7.62 36.83 180) (size 1.524 1.524) (drill 1.016) (layers "*.Cu" "*.Mask") (remove_unused_layers no)
   (roundrect_rratio 0.25) (chamfer_ratio 0.2928932188) (chamfer top_left top_right bottom_left bottom_right) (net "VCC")
   (solder_mask_margin 0.0635) (thermal_bridge_angle 0))
  (pad "C32" thru_hole roundrect (at -7.62 39.37 180) (size 1.524 1.524) (drill 1.016) (layers "*.Cu" "*.Mask") (remove_unused_layers no)
   (roundrect_rratio 0.25) (chamfer_ratio 0.2928932188) (chamfer top_left top_right bottom_left bottom_right) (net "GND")
   (solder_mask_margin 0.0635) (thermal_bridge_angle 0))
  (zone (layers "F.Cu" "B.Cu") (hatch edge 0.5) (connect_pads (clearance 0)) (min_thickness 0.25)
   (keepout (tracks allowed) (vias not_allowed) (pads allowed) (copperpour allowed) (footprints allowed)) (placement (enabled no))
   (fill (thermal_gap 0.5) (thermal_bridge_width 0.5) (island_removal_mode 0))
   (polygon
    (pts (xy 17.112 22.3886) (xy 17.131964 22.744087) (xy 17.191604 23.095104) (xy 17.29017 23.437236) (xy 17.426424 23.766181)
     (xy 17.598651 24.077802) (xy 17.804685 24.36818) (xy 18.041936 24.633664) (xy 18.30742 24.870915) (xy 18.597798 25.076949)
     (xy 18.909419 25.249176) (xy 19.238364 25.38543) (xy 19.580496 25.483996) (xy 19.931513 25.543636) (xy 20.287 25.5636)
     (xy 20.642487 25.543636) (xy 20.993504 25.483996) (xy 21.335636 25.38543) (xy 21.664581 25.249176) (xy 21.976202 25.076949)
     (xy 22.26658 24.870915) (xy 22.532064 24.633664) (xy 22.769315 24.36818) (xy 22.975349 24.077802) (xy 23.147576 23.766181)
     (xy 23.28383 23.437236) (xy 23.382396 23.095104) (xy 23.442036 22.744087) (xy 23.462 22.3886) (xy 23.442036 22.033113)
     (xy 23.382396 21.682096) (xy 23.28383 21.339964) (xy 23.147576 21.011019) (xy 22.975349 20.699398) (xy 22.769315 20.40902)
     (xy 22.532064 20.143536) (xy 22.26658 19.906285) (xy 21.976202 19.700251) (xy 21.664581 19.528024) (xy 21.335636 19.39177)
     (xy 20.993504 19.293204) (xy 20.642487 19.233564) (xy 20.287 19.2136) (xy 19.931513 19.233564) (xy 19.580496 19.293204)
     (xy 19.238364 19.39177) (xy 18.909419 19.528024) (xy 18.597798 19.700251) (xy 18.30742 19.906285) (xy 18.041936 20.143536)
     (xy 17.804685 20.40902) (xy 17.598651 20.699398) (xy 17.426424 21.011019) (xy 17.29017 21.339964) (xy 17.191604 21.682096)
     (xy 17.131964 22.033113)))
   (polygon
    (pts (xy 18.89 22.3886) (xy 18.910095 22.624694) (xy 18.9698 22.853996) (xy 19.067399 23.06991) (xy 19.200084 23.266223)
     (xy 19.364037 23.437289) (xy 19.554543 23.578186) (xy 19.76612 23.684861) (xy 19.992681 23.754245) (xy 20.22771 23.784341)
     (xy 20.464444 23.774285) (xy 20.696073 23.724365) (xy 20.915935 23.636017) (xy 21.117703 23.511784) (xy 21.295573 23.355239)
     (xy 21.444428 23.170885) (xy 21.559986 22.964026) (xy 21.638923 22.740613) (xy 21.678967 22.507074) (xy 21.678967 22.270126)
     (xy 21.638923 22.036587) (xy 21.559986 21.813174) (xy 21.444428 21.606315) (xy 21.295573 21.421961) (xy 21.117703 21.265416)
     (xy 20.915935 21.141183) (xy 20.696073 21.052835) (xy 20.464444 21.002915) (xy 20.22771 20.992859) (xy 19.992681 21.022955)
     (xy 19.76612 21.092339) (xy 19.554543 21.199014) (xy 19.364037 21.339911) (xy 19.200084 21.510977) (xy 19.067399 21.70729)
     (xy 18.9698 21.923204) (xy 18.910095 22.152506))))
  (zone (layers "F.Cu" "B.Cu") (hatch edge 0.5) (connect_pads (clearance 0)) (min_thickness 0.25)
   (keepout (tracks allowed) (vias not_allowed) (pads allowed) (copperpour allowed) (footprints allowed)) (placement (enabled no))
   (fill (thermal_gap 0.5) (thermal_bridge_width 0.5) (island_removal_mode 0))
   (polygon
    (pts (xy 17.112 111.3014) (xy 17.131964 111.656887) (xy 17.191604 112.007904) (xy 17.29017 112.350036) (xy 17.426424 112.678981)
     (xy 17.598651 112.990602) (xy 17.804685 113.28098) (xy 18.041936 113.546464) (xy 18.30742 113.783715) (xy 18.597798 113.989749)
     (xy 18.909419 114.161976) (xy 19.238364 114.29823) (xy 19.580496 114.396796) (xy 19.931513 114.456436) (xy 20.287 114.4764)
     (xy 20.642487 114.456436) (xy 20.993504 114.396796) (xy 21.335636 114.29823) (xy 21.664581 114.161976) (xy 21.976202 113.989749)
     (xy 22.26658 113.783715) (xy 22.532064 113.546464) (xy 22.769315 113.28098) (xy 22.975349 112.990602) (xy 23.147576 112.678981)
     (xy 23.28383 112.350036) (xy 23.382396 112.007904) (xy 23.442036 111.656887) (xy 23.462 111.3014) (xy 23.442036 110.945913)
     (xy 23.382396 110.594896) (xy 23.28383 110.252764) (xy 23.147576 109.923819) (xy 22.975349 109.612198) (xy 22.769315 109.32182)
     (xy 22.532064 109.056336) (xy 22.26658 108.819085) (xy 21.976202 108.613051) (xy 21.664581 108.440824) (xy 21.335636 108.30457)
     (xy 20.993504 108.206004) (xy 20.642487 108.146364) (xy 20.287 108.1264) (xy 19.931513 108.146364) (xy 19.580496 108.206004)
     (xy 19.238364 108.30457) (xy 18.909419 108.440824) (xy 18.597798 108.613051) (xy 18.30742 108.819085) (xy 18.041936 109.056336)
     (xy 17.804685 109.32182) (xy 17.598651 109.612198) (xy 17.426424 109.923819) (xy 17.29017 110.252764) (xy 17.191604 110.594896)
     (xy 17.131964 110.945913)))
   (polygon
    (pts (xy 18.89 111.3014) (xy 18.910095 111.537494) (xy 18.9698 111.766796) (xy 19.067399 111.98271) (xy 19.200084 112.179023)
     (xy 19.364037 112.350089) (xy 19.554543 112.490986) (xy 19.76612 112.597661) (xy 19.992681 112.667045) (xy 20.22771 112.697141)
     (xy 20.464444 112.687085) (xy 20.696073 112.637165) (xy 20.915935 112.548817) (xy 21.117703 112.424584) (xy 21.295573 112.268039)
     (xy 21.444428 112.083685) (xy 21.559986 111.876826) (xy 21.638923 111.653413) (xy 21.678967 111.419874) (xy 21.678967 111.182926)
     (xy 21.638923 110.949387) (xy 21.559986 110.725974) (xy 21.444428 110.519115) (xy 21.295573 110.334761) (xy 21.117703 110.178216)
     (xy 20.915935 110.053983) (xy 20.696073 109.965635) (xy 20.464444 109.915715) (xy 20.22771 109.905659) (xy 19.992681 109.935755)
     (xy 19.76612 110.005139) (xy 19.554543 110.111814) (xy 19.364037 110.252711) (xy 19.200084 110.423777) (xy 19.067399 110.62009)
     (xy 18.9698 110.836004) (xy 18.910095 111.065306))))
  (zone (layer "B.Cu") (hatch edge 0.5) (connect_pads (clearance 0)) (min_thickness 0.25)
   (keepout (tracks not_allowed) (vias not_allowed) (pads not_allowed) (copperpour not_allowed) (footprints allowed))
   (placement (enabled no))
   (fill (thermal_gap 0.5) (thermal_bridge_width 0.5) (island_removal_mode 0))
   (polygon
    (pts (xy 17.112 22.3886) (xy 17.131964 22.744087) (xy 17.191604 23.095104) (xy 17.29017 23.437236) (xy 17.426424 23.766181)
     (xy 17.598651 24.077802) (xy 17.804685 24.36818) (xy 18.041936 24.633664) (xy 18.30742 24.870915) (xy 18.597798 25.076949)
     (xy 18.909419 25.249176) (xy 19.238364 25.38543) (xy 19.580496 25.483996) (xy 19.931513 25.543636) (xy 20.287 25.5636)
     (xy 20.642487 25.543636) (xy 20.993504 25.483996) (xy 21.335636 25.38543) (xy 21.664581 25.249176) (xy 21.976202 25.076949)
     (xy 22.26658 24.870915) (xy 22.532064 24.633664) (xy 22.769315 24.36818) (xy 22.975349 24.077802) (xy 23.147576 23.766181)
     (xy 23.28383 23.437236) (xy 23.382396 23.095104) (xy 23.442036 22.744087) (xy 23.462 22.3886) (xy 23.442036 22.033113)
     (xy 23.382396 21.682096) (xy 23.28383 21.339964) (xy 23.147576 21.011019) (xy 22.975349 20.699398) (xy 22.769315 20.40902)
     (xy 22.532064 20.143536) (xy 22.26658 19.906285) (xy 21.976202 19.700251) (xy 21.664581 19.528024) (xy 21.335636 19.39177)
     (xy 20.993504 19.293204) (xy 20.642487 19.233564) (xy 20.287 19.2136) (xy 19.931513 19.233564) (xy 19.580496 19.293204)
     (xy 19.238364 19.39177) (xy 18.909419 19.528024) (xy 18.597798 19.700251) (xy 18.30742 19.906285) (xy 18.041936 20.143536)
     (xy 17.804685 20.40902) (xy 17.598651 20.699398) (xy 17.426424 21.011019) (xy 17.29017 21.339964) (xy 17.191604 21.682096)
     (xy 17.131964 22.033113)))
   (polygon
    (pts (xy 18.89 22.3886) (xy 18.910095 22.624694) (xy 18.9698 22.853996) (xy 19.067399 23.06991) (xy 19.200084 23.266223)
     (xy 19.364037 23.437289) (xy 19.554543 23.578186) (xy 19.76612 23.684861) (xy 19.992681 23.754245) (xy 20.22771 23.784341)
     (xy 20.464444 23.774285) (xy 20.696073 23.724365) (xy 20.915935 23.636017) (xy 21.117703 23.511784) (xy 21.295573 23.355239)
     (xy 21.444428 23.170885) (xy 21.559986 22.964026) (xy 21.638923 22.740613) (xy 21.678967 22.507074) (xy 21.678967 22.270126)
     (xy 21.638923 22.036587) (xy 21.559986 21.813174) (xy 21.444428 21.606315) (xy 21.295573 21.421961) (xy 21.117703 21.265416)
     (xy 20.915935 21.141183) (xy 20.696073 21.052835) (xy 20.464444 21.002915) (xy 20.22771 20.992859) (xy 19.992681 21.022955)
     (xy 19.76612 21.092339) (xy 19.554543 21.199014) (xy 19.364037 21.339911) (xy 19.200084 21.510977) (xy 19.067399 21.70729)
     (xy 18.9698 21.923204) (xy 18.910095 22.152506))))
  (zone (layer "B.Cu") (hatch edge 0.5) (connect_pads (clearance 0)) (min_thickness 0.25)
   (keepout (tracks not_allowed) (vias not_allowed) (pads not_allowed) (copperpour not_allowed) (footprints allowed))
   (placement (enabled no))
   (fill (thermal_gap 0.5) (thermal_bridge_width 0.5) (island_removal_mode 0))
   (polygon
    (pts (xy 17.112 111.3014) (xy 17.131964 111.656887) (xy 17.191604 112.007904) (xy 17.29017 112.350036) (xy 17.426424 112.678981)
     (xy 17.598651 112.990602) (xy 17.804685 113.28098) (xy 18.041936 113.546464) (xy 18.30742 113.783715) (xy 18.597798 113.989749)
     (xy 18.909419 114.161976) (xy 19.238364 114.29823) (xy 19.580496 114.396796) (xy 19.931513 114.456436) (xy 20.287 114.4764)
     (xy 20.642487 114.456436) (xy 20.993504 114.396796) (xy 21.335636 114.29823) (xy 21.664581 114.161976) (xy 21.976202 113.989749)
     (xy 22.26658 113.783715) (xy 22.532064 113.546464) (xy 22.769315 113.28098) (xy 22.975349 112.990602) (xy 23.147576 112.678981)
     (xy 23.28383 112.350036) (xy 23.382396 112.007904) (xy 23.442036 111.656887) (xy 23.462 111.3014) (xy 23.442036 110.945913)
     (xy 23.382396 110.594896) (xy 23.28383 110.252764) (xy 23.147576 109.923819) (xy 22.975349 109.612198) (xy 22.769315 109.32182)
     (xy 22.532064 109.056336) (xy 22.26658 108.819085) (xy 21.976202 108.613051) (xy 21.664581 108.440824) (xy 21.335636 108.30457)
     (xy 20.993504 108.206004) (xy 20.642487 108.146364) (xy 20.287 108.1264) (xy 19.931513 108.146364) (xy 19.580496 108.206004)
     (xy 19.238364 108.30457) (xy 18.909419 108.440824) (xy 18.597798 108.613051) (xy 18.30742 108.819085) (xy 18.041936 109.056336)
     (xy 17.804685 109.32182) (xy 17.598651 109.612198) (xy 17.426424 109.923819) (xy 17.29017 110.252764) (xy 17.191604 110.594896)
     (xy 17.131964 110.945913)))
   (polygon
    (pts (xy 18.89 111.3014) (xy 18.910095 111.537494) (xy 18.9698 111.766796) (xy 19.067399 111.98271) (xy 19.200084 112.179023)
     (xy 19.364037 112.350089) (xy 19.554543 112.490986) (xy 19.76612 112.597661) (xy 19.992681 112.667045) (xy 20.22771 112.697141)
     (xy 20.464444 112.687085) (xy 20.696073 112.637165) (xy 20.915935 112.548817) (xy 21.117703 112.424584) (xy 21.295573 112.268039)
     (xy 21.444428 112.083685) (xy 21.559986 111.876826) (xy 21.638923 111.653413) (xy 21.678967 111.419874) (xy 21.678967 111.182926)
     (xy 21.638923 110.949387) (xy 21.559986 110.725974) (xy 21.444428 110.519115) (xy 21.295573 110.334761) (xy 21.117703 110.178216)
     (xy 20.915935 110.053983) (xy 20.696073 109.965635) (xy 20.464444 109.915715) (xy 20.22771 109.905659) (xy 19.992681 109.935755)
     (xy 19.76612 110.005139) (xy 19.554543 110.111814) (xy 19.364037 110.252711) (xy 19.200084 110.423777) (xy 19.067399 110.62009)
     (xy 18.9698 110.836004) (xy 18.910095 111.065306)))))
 (gr_line (start 17.747 10.025) (end 17.747 123.995) (stroke (width 0.05) (type solid)) (layer "Edge.Cuts"))
 (gr_line (start 17.747 123.995) (end 195.527 123.995) (stroke (width 0.05) (type solid)) (layer "Edge.Cuts"))
 (gr_line (start 195.527 10.025) (end 17.747 10.025) (stroke (width 0.05) (type solid)) (layer "Edge.Cuts"))
 (gr_line (start 195.527 123.995) (end 195.527 10.025) (stroke (width 0.05) (type solid)) (layer "Edge.Cuts"))
 (segment (start 184.117 121.455) (end 182.847 120.185) (width 0.254) (layer "B.Cu") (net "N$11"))
 (segment (start 193.007 120.185) (end 191.737 121.455) (width 0.254) (layer "B.Cu") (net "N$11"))
 (segment (start 191.737 121.455) (end 184.117 121.455) (width 0.254) (layer "B.Cu") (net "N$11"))
 (segment (start 24.097 30.015) (end 22.827 30.015) (width 0.254) (layer "F.Cu") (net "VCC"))
 (segment (start 27.907 103.675) (end 156.177 103.675) (width 0.254) (layer "F.Cu") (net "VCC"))
 (segment (start 24.097 103.675) (end 24.097 30.015) (width 0.254) (layer "F.Cu") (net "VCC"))
 (segment (start 25.367 30.015) (end 24.097 30.015) (width 0.254) (layer "F.Cu") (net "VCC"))
 (segment (start 24.097 103.675) (end 22.827 103.675) (width 0.254) (layer "F.Cu") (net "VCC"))
 (segment (start 25.367 30.015) (end 27.907 30.015) (width 0.254) (layer "F.Cu") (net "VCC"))
 (segment (start 25.367 103.675) (end 24.097 103.675) (width 0.254) (layer "F.Cu") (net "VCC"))
 (segment (start 156.177 103.675) (end 172.687 120.185) (width 0.254) (layer "F.Cu") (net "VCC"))
 (segment (start 27.907 103.675) (end 25.367 103.675) (width 0.254) (layer "F.Cu") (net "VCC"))
 (segment (start 27.907 106.215) (end 25.367 106.215) (width 0.254) (layer "F.Cu") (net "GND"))
 (segment (start 25.367 106.215) (end 22.827 106.215) (width 0.254) (layer "F.Cu") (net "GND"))
 (segment (start 25.367 27.475) (end 27.907 27.475) (width 0.254) (layer "F.Cu") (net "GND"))
 (segment (start 25.367 27.475) (end 22.827 27.475) (width 0.254) (layer "F.Cu") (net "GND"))
 (segment (start 29.177 106.215) (end 29.177 28.745) (width 0.254) (layer "B.Cu") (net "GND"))
 (segment (start 29.177 28.745) (end 27.907 27.475) (width 0.254) (layer "B.Cu") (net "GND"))
 (segment (start 176.497 106.215) (end 190.467 120.185) (width 0.254) (layer "B.Cu") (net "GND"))
 (segment (start 27.907 106.215) (end 29.177 106.215) (width 0.254) (layer "B.Cu") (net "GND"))
 (segment (start 29.177 106.215) (end 176.497 106.215) (width 0.254) (layer "B.Cu") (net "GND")))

